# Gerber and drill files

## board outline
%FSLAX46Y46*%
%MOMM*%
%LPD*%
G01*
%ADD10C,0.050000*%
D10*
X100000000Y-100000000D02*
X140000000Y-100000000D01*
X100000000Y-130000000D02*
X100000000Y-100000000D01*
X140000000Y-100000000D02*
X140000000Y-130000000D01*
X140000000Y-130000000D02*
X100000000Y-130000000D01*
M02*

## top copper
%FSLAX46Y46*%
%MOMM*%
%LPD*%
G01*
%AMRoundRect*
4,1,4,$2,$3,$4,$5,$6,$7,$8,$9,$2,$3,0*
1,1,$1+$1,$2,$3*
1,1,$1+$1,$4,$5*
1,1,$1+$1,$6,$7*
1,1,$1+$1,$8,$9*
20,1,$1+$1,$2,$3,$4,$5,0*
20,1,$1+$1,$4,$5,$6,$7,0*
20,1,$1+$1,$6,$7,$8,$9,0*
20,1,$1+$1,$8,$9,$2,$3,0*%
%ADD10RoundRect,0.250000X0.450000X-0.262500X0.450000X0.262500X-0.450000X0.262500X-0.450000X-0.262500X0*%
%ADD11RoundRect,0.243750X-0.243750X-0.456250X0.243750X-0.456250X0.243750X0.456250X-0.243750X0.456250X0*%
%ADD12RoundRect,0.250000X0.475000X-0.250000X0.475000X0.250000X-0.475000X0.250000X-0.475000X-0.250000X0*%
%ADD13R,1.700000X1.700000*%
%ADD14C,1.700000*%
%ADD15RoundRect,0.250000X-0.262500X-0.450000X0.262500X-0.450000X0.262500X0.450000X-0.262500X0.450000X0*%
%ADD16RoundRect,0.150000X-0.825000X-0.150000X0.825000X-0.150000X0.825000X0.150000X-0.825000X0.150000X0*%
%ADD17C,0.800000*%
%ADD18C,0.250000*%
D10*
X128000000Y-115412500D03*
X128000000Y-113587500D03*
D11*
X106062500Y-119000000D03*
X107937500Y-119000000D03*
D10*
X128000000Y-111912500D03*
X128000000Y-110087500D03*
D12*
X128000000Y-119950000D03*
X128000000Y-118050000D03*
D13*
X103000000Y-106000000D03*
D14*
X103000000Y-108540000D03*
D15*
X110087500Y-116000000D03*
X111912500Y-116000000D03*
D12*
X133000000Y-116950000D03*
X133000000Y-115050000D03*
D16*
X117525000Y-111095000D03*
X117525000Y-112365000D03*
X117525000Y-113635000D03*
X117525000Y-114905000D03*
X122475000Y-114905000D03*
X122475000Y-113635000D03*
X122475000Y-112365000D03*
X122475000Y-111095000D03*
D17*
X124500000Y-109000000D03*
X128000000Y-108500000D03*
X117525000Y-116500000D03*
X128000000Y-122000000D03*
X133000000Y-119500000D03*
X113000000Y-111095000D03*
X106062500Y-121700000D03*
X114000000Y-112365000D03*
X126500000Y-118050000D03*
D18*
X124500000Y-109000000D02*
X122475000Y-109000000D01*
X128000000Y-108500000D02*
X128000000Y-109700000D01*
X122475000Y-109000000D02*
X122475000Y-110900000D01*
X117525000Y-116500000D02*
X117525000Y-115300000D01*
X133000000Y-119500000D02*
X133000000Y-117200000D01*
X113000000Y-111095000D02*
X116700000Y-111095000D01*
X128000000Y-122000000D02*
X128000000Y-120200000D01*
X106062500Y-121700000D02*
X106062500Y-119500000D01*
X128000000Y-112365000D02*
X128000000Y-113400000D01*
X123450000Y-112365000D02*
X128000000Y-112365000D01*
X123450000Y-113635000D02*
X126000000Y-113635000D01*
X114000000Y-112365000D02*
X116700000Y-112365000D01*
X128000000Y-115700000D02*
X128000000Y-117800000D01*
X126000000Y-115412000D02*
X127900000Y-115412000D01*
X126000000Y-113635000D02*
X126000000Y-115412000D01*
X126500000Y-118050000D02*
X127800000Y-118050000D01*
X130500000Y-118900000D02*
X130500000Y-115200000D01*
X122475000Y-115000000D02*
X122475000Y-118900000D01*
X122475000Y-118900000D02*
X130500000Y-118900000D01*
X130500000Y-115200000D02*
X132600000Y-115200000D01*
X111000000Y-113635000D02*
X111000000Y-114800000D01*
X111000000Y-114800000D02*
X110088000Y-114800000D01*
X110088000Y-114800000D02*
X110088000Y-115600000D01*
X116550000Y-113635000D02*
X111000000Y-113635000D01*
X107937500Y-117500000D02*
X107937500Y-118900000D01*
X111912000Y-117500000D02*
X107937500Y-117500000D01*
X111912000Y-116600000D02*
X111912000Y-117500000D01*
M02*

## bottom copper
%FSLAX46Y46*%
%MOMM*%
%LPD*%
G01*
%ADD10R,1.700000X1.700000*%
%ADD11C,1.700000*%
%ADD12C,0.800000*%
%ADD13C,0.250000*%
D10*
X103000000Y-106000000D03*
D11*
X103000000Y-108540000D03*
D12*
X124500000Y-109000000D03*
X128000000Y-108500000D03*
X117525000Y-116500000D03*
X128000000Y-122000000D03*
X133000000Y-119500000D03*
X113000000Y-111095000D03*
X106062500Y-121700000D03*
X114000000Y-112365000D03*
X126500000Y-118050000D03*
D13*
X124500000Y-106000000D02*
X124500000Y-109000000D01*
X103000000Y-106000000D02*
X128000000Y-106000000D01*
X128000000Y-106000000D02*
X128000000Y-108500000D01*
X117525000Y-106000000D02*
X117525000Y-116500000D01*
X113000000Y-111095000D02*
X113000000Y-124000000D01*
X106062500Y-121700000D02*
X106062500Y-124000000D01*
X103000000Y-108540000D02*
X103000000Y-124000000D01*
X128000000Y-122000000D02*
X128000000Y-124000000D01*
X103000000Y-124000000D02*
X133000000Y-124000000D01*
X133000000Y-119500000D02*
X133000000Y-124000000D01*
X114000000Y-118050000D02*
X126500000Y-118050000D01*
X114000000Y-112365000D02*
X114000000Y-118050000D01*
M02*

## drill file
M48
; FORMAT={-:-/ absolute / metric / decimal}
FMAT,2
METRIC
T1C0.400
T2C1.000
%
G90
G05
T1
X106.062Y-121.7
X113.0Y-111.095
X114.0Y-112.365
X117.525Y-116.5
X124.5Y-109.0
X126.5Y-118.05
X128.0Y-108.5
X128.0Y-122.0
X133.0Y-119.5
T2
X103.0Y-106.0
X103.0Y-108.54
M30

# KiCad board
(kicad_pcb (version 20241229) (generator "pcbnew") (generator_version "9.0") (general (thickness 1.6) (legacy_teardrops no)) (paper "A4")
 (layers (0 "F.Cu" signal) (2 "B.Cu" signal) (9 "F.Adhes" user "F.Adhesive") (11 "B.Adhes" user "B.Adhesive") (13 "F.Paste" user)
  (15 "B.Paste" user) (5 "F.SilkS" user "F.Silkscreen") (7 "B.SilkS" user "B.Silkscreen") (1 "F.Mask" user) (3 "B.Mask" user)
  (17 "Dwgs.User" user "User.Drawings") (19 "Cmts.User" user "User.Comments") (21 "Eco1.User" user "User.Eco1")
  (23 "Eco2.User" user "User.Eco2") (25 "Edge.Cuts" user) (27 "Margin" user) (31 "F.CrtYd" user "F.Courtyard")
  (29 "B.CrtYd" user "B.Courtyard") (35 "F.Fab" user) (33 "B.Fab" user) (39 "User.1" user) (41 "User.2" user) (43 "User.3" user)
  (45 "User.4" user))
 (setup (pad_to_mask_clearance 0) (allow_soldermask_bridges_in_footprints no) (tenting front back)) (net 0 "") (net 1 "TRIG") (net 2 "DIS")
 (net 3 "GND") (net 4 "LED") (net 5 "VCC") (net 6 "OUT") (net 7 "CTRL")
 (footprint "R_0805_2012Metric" (layer "F.Cu") (at 128 114.5 90)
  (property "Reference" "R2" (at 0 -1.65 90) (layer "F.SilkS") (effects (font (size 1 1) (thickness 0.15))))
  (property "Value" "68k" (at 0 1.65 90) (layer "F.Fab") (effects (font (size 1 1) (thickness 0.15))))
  (pad "1" smd roundrect (at -0.9125 0 90) (size 1.025 1.4) (layers "F.Cu" "F.Mask" "F.Paste") (roundrect_rratio 0.243902) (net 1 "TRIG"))
  (pad "2" smd roundrect (at 0.9125 0 90) (size 1.025 1.4) (layers "F.Cu" "F.Mask" "F.Paste") (roundrect_rratio 0.243902) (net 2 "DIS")))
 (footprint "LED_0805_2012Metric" (layer "F.Cu") (at 107 119)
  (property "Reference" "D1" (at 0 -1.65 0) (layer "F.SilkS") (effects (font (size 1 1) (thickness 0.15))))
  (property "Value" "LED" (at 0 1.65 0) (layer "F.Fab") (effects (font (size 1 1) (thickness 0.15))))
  (pad "1" smd roundrect (at -0.9375 0) (size 0.975 1.4) (layers "F.Cu" "F.Mask" "F.Paste") (roundrect_rratio 0.25) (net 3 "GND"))
  (pad "2" smd roundrect (at 0.9375 0) (size 0.975 1.4) (layers "F.Cu" "F.Mask" "F.Paste") (roundrect_rratio 0.25) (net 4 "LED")))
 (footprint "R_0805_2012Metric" (layer "F.Cu") (at 128 111 90)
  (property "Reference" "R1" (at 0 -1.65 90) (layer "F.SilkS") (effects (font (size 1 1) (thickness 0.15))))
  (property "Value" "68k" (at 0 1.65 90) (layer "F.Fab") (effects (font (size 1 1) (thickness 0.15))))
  (pad "1" smd roundrect (at -0.9125 0 90) (size 1.025 1.4) (layers "F.Cu" "F.Mask" "F.Paste") (roundrect_rratio 0.243902) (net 2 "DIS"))
  (pad "2" smd roundrect (at 0.9125 0 90) (size 1.025 1.4) (layers "F.Cu" "F.Mask" "F.Paste") (roundrect_rratio 0.243902) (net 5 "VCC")))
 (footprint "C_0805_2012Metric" (layer "F.Cu") (at 128 119 90)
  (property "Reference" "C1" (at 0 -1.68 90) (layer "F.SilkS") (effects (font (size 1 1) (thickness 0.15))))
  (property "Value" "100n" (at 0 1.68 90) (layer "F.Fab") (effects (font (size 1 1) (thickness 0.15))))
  (pad "1" smd roundrect (at -0.95 0 90) (size 1 1.45) (layers "F.Cu" "F.Mask" "F.Paste") (roundrect_rratio 0.25) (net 3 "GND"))
  (pad "2" smd roundrect (at 0.95 0 90) (size 1 1.45) (layers "F.Cu" "F.Mask" "F.Paste") (roundrect_rratio 0.25) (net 1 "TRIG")))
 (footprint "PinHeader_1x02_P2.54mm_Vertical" (layer "F.Cu") (at 103 106)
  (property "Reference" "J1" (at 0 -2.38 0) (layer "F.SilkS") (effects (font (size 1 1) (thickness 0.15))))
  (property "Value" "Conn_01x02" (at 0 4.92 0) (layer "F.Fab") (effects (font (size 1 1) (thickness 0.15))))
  (pad "1" thru_hole rect (at 0 0) (size 1.7 1.7) (drill 1) (layers "*.Cu" "*.Mask") (remove_unused_layers no) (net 5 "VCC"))
  (pad "2" thru_hole circle (at 0 2.54) (size 1.7 1.7) (drill 1) (layers "*.Cu" "*.Mask") (remove_unused_layers no) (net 3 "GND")))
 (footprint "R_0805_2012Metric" (layer "F.Cu") (at 111 116)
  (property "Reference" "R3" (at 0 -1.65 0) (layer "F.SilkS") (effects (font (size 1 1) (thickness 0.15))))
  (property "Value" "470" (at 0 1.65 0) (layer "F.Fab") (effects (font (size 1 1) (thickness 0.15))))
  (pad "1" smd roundrect (at -0.9125 0) (size 1.025 1.4) (layers "F.Cu" "F.Mask" "F.Paste") (roundrect_rratio 0.243902) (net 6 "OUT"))
  (pad "2" smd roundrect (at 0.9125 0) (size 1.025 1.4) (layers "F.Cu" "F.Mask" "F.Paste") (roundrect_rratio 0.243902) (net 4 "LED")))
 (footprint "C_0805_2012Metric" (layer "F.Cu") (at 133 116 90)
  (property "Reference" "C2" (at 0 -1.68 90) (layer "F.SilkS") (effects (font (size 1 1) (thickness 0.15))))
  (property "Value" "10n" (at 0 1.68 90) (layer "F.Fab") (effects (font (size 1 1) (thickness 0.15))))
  (pad "1" smd roundrect (at -0.95 0 90) (size 1 1.45) (layers "F.Cu" "F.Mask" "F.Paste") (roundrect_rratio 0.25) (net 3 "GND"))
  (pad "2" smd roundrect (at 0.95 0 90) (size 1 1.45) (layers "F.Cu" "F.Mask" "F.Paste") (roundrect_rratio 0.25) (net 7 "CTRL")))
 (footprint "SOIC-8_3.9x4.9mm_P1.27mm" (layer "F.Cu") (at 120 113)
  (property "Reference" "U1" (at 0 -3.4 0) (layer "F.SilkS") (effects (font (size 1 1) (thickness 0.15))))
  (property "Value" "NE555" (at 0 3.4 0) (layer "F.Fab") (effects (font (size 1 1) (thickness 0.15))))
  (pad "1" smd roundrect (at -2.475 -1.905) (size 1.95 0.6) (layers "F.Cu" "F.Mask" "F.Paste") (roundrect_rratio 0.25) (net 3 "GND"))
  (pad "2" smd roundrect (at -2.475 -0.635) (size 1.95 0.6) (layers "F.Cu" "F.Mask" "F.Paste") (roundrect_rratio 0.25) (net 1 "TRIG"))
  (pad "3" smd roundrect (at -2.475 0.635) (size 1.95 0.6) (layers "F.Cu" "F.Mask" "F.Paste") (roundrect_rratio 0.25) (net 6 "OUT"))
  (pad "4" smd roundrect (at -2.475 1.905) (size 1.95 0.6) (layers "F.Cu" "F.Mask" "F.Paste") (roundrect_rratio 0.25) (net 5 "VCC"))
  (pad "5" smd roundrect (at 2.475 1.905) (size 1.95 0.6) (layers "F.Cu" "F.Mask" "F.Paste") (roundrect_rratio 0.25) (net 7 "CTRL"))
  (pad "6" smd roundrect (at 2.475 0.635) (size 1.95 0.6) (layers "F.Cu" "F.Mask" "F.Paste") (roundrect_rratio 0.25) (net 1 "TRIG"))
  (pad "7" smd roundrect (at 2.475 -0.635) (size 1.95 0.6) (layers "F.Cu" "F.Mask" "F.Paste") (roundrect_rratio 0.25) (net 2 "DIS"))
  (pad "8" smd roundrect (at 2.475 -1.905) (size 1.95 0.6) (layers "F.Cu" "F.Mask" "F.Paste") (roundrect_rratio 0.25) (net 5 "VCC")))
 (gr_line (start 100 100) (end 140 100) (stroke (width 0.05) (type default)) (layer "Edge.Cuts"))
 (gr_line (start 100 130) (end 100 100) (stroke (width 0.05) (type default)) (layer "Edge.Cuts"))
 (gr_line (start 140 100) (end 140 130) (stroke (width 0.05) (type default)) (layer "Edge.Cuts"))
 (gr_line (start 140 130) (end 100 130) (stroke (width 0.05) (type default)) (layer "Edge.Cuts"))
 (segment (start 124.5 109) (end 122.475 109) (width 0.25) (layer "F.Cu") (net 5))
 (segment (start 128 108.5) (end 128 109.7) (width 0.25) (layer "F.Cu") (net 5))
 (segment (start 122.475 109) (end 122.475 110.9) (width 0.25) (layer "F.Cu") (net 5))
 (segment (start 117.525 116.5) (end 117.525 115.3) (width 0.25) (layer "F.Cu") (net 5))
 (via (at 124.5 109) (size 0.8) (drill 0.4) (layers "F.Cu" "B.Cu") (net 5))
 (via (at 128 108.5) (size 0.8) (drill 0.4) (layers "F.Cu" "B.Cu") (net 5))
 (via (at 117.525 116.5) (size 0.8) (drill 0.4) (layers "F.Cu" "B.Cu") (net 5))
 (segment (start 124.5 106) (end 124.5 109) (width 0.25) (layer "B.Cu") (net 5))
 (segment (start 103 106) (end 128 106) (width 0.25) (layer "B.Cu") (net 5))
 (segment (start 128 106) (end 128 108.5) (width 0.25) (layer "B.Cu") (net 5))
 (segment (start 117.525 106) (end 117.525 116.5) (width 0.25) (layer "B.Cu") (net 5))
 (segment (start 133 119.5) (end 133 117.2) (width 0.25) (layer "F.Cu") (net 3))
 (segment (start 113 111.095) (end 116.7 111.095) (width 0.25) (layer "F.Cu") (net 3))
 (segment (start 128 122) (end 128 120.2) (width 0.25) (layer "F.Cu") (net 3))
 (segment (start 106.0625 121.7) (end 106.0625 119.5) (width 0.25) (layer "F.Cu") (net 3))
 (via (at 128 122) (size 0.8) (drill 0.4) (layers "F.Cu" "B.Cu") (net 3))
 (via (at 133 119.5) (size 0.8) (drill 0.4) (layers "F.Cu" "B.Cu") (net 3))
 (via (at 113 111.095) (size 0.8) (drill 0.4) (layers "F.Cu" "B.Cu") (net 3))
 (via (at 106.0625 121.7) (size 0.8) (drill 0.4) (layers "F.Cu" "B.Cu") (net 3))
 (segment (start 113 111.095) (end 113 124) (width 0.25) (layer "B.Cu") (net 3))
 (segment (start 106.0625 121.7) (end 106.0625 124) (width 0.25) (layer "B.Cu") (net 3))
 (segment (start 103 108.54) (end 103 124) (width 0.25) (layer "B.Cu") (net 3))
 (segment (start 128 122) (end 128 124) (width 0.25) (layer "B.Cu") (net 3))
 (segment (start 103 124) (end 133 124) (width 0.25) (layer "B.Cu") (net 3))
 (segment (start 133 119.5) (end 133 124) (width 0.25) (layer "B.Cu") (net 3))
 (segment (start 128 112.365) (end 128 113.4) (width 0.25) (layer "F.Cu") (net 2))
 (segment (start 123.45 112.365) (end 128 112.365) (width 0.25) (layer "F.Cu") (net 2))
 (segment (start 123.45 113.635) (end 126 113.635) (width 0.25) (layer "F.Cu") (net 1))
 (segment (start 114 112.365) (end 116.7 112.365) (width 0.25) (layer "F.Cu") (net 1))
 (segment (start 128 115.7) (end 128 117.8) (width 0.25) (layer "F.Cu") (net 1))
 (segment (start 126 115.412) (end 127.9 115.412) (width 0.25) (layer "F.Cu") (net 1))
 (segment (start 126 113.635) (end 126 115.412) (width 0.25) (layer "F.Cu") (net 1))
 (segment (start 126.5 118.05) (end 127.8 118.05) (width 0.25) (layer "F.Cu") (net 1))
 (via (at 114 112.365) (size 0.8) (drill 0.4) (layers "F.Cu" "B.Cu") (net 1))
 (via (at 126.5 118.05) (size 0.8) (drill 0.4) (layers "F.Cu" "B.Cu") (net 1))
 (segment (start 114 118.05) (end 126.5 118.05) (width 0.25) (layer "B.Cu") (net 1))
 (segment (start 114 112.365) (end 114 118.05) (width 0.25) (layer "B.Cu") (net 1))
 (segment (start 130.5 118.9) (end 130.5 115.2) (width 0.25) (layer "F.Cu") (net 7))
 (segment (start 122.475 115) (end 122.475 118.9) (width 0.25) (layer "F.Cu") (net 7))
 (segment (start 122.475 118.9) (end 130.5 118.9) (width 0.25) (layer "F.Cu") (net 7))
 (segment (start 130.5 115.2) (end 132.6 115.2) (width 0.25) (layer "F.Cu") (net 7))
 (segment (start 111 113.635) (end 111 114.8) (width 0.25) (layer "F.Cu") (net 6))
 (segment (start 111 114.8) (end 110.088 114.8) (width 0.25) (layer "F.Cu") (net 6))
 (segment (start 110.088 114.8) (end 110.088 115.6) (width 0.25) (layer "F.Cu") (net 6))
 (segment (start 116.55 113.635) (end 111 113.635) (width 0.25) (layer "F.Cu") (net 6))
 (segment (start 107.9375 117.5) (end 107.9375 118.9) (width 0.25) (layer "F.Cu") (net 4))
 (segment (start 111.912 117.5) (end 107.9375 117.5) (width 0.25) (layer "F.Cu") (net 4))
 (segment (start 111.912 116.6) (end 111.912 117.5) (width 0.25) (layer "F.Cu") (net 4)))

